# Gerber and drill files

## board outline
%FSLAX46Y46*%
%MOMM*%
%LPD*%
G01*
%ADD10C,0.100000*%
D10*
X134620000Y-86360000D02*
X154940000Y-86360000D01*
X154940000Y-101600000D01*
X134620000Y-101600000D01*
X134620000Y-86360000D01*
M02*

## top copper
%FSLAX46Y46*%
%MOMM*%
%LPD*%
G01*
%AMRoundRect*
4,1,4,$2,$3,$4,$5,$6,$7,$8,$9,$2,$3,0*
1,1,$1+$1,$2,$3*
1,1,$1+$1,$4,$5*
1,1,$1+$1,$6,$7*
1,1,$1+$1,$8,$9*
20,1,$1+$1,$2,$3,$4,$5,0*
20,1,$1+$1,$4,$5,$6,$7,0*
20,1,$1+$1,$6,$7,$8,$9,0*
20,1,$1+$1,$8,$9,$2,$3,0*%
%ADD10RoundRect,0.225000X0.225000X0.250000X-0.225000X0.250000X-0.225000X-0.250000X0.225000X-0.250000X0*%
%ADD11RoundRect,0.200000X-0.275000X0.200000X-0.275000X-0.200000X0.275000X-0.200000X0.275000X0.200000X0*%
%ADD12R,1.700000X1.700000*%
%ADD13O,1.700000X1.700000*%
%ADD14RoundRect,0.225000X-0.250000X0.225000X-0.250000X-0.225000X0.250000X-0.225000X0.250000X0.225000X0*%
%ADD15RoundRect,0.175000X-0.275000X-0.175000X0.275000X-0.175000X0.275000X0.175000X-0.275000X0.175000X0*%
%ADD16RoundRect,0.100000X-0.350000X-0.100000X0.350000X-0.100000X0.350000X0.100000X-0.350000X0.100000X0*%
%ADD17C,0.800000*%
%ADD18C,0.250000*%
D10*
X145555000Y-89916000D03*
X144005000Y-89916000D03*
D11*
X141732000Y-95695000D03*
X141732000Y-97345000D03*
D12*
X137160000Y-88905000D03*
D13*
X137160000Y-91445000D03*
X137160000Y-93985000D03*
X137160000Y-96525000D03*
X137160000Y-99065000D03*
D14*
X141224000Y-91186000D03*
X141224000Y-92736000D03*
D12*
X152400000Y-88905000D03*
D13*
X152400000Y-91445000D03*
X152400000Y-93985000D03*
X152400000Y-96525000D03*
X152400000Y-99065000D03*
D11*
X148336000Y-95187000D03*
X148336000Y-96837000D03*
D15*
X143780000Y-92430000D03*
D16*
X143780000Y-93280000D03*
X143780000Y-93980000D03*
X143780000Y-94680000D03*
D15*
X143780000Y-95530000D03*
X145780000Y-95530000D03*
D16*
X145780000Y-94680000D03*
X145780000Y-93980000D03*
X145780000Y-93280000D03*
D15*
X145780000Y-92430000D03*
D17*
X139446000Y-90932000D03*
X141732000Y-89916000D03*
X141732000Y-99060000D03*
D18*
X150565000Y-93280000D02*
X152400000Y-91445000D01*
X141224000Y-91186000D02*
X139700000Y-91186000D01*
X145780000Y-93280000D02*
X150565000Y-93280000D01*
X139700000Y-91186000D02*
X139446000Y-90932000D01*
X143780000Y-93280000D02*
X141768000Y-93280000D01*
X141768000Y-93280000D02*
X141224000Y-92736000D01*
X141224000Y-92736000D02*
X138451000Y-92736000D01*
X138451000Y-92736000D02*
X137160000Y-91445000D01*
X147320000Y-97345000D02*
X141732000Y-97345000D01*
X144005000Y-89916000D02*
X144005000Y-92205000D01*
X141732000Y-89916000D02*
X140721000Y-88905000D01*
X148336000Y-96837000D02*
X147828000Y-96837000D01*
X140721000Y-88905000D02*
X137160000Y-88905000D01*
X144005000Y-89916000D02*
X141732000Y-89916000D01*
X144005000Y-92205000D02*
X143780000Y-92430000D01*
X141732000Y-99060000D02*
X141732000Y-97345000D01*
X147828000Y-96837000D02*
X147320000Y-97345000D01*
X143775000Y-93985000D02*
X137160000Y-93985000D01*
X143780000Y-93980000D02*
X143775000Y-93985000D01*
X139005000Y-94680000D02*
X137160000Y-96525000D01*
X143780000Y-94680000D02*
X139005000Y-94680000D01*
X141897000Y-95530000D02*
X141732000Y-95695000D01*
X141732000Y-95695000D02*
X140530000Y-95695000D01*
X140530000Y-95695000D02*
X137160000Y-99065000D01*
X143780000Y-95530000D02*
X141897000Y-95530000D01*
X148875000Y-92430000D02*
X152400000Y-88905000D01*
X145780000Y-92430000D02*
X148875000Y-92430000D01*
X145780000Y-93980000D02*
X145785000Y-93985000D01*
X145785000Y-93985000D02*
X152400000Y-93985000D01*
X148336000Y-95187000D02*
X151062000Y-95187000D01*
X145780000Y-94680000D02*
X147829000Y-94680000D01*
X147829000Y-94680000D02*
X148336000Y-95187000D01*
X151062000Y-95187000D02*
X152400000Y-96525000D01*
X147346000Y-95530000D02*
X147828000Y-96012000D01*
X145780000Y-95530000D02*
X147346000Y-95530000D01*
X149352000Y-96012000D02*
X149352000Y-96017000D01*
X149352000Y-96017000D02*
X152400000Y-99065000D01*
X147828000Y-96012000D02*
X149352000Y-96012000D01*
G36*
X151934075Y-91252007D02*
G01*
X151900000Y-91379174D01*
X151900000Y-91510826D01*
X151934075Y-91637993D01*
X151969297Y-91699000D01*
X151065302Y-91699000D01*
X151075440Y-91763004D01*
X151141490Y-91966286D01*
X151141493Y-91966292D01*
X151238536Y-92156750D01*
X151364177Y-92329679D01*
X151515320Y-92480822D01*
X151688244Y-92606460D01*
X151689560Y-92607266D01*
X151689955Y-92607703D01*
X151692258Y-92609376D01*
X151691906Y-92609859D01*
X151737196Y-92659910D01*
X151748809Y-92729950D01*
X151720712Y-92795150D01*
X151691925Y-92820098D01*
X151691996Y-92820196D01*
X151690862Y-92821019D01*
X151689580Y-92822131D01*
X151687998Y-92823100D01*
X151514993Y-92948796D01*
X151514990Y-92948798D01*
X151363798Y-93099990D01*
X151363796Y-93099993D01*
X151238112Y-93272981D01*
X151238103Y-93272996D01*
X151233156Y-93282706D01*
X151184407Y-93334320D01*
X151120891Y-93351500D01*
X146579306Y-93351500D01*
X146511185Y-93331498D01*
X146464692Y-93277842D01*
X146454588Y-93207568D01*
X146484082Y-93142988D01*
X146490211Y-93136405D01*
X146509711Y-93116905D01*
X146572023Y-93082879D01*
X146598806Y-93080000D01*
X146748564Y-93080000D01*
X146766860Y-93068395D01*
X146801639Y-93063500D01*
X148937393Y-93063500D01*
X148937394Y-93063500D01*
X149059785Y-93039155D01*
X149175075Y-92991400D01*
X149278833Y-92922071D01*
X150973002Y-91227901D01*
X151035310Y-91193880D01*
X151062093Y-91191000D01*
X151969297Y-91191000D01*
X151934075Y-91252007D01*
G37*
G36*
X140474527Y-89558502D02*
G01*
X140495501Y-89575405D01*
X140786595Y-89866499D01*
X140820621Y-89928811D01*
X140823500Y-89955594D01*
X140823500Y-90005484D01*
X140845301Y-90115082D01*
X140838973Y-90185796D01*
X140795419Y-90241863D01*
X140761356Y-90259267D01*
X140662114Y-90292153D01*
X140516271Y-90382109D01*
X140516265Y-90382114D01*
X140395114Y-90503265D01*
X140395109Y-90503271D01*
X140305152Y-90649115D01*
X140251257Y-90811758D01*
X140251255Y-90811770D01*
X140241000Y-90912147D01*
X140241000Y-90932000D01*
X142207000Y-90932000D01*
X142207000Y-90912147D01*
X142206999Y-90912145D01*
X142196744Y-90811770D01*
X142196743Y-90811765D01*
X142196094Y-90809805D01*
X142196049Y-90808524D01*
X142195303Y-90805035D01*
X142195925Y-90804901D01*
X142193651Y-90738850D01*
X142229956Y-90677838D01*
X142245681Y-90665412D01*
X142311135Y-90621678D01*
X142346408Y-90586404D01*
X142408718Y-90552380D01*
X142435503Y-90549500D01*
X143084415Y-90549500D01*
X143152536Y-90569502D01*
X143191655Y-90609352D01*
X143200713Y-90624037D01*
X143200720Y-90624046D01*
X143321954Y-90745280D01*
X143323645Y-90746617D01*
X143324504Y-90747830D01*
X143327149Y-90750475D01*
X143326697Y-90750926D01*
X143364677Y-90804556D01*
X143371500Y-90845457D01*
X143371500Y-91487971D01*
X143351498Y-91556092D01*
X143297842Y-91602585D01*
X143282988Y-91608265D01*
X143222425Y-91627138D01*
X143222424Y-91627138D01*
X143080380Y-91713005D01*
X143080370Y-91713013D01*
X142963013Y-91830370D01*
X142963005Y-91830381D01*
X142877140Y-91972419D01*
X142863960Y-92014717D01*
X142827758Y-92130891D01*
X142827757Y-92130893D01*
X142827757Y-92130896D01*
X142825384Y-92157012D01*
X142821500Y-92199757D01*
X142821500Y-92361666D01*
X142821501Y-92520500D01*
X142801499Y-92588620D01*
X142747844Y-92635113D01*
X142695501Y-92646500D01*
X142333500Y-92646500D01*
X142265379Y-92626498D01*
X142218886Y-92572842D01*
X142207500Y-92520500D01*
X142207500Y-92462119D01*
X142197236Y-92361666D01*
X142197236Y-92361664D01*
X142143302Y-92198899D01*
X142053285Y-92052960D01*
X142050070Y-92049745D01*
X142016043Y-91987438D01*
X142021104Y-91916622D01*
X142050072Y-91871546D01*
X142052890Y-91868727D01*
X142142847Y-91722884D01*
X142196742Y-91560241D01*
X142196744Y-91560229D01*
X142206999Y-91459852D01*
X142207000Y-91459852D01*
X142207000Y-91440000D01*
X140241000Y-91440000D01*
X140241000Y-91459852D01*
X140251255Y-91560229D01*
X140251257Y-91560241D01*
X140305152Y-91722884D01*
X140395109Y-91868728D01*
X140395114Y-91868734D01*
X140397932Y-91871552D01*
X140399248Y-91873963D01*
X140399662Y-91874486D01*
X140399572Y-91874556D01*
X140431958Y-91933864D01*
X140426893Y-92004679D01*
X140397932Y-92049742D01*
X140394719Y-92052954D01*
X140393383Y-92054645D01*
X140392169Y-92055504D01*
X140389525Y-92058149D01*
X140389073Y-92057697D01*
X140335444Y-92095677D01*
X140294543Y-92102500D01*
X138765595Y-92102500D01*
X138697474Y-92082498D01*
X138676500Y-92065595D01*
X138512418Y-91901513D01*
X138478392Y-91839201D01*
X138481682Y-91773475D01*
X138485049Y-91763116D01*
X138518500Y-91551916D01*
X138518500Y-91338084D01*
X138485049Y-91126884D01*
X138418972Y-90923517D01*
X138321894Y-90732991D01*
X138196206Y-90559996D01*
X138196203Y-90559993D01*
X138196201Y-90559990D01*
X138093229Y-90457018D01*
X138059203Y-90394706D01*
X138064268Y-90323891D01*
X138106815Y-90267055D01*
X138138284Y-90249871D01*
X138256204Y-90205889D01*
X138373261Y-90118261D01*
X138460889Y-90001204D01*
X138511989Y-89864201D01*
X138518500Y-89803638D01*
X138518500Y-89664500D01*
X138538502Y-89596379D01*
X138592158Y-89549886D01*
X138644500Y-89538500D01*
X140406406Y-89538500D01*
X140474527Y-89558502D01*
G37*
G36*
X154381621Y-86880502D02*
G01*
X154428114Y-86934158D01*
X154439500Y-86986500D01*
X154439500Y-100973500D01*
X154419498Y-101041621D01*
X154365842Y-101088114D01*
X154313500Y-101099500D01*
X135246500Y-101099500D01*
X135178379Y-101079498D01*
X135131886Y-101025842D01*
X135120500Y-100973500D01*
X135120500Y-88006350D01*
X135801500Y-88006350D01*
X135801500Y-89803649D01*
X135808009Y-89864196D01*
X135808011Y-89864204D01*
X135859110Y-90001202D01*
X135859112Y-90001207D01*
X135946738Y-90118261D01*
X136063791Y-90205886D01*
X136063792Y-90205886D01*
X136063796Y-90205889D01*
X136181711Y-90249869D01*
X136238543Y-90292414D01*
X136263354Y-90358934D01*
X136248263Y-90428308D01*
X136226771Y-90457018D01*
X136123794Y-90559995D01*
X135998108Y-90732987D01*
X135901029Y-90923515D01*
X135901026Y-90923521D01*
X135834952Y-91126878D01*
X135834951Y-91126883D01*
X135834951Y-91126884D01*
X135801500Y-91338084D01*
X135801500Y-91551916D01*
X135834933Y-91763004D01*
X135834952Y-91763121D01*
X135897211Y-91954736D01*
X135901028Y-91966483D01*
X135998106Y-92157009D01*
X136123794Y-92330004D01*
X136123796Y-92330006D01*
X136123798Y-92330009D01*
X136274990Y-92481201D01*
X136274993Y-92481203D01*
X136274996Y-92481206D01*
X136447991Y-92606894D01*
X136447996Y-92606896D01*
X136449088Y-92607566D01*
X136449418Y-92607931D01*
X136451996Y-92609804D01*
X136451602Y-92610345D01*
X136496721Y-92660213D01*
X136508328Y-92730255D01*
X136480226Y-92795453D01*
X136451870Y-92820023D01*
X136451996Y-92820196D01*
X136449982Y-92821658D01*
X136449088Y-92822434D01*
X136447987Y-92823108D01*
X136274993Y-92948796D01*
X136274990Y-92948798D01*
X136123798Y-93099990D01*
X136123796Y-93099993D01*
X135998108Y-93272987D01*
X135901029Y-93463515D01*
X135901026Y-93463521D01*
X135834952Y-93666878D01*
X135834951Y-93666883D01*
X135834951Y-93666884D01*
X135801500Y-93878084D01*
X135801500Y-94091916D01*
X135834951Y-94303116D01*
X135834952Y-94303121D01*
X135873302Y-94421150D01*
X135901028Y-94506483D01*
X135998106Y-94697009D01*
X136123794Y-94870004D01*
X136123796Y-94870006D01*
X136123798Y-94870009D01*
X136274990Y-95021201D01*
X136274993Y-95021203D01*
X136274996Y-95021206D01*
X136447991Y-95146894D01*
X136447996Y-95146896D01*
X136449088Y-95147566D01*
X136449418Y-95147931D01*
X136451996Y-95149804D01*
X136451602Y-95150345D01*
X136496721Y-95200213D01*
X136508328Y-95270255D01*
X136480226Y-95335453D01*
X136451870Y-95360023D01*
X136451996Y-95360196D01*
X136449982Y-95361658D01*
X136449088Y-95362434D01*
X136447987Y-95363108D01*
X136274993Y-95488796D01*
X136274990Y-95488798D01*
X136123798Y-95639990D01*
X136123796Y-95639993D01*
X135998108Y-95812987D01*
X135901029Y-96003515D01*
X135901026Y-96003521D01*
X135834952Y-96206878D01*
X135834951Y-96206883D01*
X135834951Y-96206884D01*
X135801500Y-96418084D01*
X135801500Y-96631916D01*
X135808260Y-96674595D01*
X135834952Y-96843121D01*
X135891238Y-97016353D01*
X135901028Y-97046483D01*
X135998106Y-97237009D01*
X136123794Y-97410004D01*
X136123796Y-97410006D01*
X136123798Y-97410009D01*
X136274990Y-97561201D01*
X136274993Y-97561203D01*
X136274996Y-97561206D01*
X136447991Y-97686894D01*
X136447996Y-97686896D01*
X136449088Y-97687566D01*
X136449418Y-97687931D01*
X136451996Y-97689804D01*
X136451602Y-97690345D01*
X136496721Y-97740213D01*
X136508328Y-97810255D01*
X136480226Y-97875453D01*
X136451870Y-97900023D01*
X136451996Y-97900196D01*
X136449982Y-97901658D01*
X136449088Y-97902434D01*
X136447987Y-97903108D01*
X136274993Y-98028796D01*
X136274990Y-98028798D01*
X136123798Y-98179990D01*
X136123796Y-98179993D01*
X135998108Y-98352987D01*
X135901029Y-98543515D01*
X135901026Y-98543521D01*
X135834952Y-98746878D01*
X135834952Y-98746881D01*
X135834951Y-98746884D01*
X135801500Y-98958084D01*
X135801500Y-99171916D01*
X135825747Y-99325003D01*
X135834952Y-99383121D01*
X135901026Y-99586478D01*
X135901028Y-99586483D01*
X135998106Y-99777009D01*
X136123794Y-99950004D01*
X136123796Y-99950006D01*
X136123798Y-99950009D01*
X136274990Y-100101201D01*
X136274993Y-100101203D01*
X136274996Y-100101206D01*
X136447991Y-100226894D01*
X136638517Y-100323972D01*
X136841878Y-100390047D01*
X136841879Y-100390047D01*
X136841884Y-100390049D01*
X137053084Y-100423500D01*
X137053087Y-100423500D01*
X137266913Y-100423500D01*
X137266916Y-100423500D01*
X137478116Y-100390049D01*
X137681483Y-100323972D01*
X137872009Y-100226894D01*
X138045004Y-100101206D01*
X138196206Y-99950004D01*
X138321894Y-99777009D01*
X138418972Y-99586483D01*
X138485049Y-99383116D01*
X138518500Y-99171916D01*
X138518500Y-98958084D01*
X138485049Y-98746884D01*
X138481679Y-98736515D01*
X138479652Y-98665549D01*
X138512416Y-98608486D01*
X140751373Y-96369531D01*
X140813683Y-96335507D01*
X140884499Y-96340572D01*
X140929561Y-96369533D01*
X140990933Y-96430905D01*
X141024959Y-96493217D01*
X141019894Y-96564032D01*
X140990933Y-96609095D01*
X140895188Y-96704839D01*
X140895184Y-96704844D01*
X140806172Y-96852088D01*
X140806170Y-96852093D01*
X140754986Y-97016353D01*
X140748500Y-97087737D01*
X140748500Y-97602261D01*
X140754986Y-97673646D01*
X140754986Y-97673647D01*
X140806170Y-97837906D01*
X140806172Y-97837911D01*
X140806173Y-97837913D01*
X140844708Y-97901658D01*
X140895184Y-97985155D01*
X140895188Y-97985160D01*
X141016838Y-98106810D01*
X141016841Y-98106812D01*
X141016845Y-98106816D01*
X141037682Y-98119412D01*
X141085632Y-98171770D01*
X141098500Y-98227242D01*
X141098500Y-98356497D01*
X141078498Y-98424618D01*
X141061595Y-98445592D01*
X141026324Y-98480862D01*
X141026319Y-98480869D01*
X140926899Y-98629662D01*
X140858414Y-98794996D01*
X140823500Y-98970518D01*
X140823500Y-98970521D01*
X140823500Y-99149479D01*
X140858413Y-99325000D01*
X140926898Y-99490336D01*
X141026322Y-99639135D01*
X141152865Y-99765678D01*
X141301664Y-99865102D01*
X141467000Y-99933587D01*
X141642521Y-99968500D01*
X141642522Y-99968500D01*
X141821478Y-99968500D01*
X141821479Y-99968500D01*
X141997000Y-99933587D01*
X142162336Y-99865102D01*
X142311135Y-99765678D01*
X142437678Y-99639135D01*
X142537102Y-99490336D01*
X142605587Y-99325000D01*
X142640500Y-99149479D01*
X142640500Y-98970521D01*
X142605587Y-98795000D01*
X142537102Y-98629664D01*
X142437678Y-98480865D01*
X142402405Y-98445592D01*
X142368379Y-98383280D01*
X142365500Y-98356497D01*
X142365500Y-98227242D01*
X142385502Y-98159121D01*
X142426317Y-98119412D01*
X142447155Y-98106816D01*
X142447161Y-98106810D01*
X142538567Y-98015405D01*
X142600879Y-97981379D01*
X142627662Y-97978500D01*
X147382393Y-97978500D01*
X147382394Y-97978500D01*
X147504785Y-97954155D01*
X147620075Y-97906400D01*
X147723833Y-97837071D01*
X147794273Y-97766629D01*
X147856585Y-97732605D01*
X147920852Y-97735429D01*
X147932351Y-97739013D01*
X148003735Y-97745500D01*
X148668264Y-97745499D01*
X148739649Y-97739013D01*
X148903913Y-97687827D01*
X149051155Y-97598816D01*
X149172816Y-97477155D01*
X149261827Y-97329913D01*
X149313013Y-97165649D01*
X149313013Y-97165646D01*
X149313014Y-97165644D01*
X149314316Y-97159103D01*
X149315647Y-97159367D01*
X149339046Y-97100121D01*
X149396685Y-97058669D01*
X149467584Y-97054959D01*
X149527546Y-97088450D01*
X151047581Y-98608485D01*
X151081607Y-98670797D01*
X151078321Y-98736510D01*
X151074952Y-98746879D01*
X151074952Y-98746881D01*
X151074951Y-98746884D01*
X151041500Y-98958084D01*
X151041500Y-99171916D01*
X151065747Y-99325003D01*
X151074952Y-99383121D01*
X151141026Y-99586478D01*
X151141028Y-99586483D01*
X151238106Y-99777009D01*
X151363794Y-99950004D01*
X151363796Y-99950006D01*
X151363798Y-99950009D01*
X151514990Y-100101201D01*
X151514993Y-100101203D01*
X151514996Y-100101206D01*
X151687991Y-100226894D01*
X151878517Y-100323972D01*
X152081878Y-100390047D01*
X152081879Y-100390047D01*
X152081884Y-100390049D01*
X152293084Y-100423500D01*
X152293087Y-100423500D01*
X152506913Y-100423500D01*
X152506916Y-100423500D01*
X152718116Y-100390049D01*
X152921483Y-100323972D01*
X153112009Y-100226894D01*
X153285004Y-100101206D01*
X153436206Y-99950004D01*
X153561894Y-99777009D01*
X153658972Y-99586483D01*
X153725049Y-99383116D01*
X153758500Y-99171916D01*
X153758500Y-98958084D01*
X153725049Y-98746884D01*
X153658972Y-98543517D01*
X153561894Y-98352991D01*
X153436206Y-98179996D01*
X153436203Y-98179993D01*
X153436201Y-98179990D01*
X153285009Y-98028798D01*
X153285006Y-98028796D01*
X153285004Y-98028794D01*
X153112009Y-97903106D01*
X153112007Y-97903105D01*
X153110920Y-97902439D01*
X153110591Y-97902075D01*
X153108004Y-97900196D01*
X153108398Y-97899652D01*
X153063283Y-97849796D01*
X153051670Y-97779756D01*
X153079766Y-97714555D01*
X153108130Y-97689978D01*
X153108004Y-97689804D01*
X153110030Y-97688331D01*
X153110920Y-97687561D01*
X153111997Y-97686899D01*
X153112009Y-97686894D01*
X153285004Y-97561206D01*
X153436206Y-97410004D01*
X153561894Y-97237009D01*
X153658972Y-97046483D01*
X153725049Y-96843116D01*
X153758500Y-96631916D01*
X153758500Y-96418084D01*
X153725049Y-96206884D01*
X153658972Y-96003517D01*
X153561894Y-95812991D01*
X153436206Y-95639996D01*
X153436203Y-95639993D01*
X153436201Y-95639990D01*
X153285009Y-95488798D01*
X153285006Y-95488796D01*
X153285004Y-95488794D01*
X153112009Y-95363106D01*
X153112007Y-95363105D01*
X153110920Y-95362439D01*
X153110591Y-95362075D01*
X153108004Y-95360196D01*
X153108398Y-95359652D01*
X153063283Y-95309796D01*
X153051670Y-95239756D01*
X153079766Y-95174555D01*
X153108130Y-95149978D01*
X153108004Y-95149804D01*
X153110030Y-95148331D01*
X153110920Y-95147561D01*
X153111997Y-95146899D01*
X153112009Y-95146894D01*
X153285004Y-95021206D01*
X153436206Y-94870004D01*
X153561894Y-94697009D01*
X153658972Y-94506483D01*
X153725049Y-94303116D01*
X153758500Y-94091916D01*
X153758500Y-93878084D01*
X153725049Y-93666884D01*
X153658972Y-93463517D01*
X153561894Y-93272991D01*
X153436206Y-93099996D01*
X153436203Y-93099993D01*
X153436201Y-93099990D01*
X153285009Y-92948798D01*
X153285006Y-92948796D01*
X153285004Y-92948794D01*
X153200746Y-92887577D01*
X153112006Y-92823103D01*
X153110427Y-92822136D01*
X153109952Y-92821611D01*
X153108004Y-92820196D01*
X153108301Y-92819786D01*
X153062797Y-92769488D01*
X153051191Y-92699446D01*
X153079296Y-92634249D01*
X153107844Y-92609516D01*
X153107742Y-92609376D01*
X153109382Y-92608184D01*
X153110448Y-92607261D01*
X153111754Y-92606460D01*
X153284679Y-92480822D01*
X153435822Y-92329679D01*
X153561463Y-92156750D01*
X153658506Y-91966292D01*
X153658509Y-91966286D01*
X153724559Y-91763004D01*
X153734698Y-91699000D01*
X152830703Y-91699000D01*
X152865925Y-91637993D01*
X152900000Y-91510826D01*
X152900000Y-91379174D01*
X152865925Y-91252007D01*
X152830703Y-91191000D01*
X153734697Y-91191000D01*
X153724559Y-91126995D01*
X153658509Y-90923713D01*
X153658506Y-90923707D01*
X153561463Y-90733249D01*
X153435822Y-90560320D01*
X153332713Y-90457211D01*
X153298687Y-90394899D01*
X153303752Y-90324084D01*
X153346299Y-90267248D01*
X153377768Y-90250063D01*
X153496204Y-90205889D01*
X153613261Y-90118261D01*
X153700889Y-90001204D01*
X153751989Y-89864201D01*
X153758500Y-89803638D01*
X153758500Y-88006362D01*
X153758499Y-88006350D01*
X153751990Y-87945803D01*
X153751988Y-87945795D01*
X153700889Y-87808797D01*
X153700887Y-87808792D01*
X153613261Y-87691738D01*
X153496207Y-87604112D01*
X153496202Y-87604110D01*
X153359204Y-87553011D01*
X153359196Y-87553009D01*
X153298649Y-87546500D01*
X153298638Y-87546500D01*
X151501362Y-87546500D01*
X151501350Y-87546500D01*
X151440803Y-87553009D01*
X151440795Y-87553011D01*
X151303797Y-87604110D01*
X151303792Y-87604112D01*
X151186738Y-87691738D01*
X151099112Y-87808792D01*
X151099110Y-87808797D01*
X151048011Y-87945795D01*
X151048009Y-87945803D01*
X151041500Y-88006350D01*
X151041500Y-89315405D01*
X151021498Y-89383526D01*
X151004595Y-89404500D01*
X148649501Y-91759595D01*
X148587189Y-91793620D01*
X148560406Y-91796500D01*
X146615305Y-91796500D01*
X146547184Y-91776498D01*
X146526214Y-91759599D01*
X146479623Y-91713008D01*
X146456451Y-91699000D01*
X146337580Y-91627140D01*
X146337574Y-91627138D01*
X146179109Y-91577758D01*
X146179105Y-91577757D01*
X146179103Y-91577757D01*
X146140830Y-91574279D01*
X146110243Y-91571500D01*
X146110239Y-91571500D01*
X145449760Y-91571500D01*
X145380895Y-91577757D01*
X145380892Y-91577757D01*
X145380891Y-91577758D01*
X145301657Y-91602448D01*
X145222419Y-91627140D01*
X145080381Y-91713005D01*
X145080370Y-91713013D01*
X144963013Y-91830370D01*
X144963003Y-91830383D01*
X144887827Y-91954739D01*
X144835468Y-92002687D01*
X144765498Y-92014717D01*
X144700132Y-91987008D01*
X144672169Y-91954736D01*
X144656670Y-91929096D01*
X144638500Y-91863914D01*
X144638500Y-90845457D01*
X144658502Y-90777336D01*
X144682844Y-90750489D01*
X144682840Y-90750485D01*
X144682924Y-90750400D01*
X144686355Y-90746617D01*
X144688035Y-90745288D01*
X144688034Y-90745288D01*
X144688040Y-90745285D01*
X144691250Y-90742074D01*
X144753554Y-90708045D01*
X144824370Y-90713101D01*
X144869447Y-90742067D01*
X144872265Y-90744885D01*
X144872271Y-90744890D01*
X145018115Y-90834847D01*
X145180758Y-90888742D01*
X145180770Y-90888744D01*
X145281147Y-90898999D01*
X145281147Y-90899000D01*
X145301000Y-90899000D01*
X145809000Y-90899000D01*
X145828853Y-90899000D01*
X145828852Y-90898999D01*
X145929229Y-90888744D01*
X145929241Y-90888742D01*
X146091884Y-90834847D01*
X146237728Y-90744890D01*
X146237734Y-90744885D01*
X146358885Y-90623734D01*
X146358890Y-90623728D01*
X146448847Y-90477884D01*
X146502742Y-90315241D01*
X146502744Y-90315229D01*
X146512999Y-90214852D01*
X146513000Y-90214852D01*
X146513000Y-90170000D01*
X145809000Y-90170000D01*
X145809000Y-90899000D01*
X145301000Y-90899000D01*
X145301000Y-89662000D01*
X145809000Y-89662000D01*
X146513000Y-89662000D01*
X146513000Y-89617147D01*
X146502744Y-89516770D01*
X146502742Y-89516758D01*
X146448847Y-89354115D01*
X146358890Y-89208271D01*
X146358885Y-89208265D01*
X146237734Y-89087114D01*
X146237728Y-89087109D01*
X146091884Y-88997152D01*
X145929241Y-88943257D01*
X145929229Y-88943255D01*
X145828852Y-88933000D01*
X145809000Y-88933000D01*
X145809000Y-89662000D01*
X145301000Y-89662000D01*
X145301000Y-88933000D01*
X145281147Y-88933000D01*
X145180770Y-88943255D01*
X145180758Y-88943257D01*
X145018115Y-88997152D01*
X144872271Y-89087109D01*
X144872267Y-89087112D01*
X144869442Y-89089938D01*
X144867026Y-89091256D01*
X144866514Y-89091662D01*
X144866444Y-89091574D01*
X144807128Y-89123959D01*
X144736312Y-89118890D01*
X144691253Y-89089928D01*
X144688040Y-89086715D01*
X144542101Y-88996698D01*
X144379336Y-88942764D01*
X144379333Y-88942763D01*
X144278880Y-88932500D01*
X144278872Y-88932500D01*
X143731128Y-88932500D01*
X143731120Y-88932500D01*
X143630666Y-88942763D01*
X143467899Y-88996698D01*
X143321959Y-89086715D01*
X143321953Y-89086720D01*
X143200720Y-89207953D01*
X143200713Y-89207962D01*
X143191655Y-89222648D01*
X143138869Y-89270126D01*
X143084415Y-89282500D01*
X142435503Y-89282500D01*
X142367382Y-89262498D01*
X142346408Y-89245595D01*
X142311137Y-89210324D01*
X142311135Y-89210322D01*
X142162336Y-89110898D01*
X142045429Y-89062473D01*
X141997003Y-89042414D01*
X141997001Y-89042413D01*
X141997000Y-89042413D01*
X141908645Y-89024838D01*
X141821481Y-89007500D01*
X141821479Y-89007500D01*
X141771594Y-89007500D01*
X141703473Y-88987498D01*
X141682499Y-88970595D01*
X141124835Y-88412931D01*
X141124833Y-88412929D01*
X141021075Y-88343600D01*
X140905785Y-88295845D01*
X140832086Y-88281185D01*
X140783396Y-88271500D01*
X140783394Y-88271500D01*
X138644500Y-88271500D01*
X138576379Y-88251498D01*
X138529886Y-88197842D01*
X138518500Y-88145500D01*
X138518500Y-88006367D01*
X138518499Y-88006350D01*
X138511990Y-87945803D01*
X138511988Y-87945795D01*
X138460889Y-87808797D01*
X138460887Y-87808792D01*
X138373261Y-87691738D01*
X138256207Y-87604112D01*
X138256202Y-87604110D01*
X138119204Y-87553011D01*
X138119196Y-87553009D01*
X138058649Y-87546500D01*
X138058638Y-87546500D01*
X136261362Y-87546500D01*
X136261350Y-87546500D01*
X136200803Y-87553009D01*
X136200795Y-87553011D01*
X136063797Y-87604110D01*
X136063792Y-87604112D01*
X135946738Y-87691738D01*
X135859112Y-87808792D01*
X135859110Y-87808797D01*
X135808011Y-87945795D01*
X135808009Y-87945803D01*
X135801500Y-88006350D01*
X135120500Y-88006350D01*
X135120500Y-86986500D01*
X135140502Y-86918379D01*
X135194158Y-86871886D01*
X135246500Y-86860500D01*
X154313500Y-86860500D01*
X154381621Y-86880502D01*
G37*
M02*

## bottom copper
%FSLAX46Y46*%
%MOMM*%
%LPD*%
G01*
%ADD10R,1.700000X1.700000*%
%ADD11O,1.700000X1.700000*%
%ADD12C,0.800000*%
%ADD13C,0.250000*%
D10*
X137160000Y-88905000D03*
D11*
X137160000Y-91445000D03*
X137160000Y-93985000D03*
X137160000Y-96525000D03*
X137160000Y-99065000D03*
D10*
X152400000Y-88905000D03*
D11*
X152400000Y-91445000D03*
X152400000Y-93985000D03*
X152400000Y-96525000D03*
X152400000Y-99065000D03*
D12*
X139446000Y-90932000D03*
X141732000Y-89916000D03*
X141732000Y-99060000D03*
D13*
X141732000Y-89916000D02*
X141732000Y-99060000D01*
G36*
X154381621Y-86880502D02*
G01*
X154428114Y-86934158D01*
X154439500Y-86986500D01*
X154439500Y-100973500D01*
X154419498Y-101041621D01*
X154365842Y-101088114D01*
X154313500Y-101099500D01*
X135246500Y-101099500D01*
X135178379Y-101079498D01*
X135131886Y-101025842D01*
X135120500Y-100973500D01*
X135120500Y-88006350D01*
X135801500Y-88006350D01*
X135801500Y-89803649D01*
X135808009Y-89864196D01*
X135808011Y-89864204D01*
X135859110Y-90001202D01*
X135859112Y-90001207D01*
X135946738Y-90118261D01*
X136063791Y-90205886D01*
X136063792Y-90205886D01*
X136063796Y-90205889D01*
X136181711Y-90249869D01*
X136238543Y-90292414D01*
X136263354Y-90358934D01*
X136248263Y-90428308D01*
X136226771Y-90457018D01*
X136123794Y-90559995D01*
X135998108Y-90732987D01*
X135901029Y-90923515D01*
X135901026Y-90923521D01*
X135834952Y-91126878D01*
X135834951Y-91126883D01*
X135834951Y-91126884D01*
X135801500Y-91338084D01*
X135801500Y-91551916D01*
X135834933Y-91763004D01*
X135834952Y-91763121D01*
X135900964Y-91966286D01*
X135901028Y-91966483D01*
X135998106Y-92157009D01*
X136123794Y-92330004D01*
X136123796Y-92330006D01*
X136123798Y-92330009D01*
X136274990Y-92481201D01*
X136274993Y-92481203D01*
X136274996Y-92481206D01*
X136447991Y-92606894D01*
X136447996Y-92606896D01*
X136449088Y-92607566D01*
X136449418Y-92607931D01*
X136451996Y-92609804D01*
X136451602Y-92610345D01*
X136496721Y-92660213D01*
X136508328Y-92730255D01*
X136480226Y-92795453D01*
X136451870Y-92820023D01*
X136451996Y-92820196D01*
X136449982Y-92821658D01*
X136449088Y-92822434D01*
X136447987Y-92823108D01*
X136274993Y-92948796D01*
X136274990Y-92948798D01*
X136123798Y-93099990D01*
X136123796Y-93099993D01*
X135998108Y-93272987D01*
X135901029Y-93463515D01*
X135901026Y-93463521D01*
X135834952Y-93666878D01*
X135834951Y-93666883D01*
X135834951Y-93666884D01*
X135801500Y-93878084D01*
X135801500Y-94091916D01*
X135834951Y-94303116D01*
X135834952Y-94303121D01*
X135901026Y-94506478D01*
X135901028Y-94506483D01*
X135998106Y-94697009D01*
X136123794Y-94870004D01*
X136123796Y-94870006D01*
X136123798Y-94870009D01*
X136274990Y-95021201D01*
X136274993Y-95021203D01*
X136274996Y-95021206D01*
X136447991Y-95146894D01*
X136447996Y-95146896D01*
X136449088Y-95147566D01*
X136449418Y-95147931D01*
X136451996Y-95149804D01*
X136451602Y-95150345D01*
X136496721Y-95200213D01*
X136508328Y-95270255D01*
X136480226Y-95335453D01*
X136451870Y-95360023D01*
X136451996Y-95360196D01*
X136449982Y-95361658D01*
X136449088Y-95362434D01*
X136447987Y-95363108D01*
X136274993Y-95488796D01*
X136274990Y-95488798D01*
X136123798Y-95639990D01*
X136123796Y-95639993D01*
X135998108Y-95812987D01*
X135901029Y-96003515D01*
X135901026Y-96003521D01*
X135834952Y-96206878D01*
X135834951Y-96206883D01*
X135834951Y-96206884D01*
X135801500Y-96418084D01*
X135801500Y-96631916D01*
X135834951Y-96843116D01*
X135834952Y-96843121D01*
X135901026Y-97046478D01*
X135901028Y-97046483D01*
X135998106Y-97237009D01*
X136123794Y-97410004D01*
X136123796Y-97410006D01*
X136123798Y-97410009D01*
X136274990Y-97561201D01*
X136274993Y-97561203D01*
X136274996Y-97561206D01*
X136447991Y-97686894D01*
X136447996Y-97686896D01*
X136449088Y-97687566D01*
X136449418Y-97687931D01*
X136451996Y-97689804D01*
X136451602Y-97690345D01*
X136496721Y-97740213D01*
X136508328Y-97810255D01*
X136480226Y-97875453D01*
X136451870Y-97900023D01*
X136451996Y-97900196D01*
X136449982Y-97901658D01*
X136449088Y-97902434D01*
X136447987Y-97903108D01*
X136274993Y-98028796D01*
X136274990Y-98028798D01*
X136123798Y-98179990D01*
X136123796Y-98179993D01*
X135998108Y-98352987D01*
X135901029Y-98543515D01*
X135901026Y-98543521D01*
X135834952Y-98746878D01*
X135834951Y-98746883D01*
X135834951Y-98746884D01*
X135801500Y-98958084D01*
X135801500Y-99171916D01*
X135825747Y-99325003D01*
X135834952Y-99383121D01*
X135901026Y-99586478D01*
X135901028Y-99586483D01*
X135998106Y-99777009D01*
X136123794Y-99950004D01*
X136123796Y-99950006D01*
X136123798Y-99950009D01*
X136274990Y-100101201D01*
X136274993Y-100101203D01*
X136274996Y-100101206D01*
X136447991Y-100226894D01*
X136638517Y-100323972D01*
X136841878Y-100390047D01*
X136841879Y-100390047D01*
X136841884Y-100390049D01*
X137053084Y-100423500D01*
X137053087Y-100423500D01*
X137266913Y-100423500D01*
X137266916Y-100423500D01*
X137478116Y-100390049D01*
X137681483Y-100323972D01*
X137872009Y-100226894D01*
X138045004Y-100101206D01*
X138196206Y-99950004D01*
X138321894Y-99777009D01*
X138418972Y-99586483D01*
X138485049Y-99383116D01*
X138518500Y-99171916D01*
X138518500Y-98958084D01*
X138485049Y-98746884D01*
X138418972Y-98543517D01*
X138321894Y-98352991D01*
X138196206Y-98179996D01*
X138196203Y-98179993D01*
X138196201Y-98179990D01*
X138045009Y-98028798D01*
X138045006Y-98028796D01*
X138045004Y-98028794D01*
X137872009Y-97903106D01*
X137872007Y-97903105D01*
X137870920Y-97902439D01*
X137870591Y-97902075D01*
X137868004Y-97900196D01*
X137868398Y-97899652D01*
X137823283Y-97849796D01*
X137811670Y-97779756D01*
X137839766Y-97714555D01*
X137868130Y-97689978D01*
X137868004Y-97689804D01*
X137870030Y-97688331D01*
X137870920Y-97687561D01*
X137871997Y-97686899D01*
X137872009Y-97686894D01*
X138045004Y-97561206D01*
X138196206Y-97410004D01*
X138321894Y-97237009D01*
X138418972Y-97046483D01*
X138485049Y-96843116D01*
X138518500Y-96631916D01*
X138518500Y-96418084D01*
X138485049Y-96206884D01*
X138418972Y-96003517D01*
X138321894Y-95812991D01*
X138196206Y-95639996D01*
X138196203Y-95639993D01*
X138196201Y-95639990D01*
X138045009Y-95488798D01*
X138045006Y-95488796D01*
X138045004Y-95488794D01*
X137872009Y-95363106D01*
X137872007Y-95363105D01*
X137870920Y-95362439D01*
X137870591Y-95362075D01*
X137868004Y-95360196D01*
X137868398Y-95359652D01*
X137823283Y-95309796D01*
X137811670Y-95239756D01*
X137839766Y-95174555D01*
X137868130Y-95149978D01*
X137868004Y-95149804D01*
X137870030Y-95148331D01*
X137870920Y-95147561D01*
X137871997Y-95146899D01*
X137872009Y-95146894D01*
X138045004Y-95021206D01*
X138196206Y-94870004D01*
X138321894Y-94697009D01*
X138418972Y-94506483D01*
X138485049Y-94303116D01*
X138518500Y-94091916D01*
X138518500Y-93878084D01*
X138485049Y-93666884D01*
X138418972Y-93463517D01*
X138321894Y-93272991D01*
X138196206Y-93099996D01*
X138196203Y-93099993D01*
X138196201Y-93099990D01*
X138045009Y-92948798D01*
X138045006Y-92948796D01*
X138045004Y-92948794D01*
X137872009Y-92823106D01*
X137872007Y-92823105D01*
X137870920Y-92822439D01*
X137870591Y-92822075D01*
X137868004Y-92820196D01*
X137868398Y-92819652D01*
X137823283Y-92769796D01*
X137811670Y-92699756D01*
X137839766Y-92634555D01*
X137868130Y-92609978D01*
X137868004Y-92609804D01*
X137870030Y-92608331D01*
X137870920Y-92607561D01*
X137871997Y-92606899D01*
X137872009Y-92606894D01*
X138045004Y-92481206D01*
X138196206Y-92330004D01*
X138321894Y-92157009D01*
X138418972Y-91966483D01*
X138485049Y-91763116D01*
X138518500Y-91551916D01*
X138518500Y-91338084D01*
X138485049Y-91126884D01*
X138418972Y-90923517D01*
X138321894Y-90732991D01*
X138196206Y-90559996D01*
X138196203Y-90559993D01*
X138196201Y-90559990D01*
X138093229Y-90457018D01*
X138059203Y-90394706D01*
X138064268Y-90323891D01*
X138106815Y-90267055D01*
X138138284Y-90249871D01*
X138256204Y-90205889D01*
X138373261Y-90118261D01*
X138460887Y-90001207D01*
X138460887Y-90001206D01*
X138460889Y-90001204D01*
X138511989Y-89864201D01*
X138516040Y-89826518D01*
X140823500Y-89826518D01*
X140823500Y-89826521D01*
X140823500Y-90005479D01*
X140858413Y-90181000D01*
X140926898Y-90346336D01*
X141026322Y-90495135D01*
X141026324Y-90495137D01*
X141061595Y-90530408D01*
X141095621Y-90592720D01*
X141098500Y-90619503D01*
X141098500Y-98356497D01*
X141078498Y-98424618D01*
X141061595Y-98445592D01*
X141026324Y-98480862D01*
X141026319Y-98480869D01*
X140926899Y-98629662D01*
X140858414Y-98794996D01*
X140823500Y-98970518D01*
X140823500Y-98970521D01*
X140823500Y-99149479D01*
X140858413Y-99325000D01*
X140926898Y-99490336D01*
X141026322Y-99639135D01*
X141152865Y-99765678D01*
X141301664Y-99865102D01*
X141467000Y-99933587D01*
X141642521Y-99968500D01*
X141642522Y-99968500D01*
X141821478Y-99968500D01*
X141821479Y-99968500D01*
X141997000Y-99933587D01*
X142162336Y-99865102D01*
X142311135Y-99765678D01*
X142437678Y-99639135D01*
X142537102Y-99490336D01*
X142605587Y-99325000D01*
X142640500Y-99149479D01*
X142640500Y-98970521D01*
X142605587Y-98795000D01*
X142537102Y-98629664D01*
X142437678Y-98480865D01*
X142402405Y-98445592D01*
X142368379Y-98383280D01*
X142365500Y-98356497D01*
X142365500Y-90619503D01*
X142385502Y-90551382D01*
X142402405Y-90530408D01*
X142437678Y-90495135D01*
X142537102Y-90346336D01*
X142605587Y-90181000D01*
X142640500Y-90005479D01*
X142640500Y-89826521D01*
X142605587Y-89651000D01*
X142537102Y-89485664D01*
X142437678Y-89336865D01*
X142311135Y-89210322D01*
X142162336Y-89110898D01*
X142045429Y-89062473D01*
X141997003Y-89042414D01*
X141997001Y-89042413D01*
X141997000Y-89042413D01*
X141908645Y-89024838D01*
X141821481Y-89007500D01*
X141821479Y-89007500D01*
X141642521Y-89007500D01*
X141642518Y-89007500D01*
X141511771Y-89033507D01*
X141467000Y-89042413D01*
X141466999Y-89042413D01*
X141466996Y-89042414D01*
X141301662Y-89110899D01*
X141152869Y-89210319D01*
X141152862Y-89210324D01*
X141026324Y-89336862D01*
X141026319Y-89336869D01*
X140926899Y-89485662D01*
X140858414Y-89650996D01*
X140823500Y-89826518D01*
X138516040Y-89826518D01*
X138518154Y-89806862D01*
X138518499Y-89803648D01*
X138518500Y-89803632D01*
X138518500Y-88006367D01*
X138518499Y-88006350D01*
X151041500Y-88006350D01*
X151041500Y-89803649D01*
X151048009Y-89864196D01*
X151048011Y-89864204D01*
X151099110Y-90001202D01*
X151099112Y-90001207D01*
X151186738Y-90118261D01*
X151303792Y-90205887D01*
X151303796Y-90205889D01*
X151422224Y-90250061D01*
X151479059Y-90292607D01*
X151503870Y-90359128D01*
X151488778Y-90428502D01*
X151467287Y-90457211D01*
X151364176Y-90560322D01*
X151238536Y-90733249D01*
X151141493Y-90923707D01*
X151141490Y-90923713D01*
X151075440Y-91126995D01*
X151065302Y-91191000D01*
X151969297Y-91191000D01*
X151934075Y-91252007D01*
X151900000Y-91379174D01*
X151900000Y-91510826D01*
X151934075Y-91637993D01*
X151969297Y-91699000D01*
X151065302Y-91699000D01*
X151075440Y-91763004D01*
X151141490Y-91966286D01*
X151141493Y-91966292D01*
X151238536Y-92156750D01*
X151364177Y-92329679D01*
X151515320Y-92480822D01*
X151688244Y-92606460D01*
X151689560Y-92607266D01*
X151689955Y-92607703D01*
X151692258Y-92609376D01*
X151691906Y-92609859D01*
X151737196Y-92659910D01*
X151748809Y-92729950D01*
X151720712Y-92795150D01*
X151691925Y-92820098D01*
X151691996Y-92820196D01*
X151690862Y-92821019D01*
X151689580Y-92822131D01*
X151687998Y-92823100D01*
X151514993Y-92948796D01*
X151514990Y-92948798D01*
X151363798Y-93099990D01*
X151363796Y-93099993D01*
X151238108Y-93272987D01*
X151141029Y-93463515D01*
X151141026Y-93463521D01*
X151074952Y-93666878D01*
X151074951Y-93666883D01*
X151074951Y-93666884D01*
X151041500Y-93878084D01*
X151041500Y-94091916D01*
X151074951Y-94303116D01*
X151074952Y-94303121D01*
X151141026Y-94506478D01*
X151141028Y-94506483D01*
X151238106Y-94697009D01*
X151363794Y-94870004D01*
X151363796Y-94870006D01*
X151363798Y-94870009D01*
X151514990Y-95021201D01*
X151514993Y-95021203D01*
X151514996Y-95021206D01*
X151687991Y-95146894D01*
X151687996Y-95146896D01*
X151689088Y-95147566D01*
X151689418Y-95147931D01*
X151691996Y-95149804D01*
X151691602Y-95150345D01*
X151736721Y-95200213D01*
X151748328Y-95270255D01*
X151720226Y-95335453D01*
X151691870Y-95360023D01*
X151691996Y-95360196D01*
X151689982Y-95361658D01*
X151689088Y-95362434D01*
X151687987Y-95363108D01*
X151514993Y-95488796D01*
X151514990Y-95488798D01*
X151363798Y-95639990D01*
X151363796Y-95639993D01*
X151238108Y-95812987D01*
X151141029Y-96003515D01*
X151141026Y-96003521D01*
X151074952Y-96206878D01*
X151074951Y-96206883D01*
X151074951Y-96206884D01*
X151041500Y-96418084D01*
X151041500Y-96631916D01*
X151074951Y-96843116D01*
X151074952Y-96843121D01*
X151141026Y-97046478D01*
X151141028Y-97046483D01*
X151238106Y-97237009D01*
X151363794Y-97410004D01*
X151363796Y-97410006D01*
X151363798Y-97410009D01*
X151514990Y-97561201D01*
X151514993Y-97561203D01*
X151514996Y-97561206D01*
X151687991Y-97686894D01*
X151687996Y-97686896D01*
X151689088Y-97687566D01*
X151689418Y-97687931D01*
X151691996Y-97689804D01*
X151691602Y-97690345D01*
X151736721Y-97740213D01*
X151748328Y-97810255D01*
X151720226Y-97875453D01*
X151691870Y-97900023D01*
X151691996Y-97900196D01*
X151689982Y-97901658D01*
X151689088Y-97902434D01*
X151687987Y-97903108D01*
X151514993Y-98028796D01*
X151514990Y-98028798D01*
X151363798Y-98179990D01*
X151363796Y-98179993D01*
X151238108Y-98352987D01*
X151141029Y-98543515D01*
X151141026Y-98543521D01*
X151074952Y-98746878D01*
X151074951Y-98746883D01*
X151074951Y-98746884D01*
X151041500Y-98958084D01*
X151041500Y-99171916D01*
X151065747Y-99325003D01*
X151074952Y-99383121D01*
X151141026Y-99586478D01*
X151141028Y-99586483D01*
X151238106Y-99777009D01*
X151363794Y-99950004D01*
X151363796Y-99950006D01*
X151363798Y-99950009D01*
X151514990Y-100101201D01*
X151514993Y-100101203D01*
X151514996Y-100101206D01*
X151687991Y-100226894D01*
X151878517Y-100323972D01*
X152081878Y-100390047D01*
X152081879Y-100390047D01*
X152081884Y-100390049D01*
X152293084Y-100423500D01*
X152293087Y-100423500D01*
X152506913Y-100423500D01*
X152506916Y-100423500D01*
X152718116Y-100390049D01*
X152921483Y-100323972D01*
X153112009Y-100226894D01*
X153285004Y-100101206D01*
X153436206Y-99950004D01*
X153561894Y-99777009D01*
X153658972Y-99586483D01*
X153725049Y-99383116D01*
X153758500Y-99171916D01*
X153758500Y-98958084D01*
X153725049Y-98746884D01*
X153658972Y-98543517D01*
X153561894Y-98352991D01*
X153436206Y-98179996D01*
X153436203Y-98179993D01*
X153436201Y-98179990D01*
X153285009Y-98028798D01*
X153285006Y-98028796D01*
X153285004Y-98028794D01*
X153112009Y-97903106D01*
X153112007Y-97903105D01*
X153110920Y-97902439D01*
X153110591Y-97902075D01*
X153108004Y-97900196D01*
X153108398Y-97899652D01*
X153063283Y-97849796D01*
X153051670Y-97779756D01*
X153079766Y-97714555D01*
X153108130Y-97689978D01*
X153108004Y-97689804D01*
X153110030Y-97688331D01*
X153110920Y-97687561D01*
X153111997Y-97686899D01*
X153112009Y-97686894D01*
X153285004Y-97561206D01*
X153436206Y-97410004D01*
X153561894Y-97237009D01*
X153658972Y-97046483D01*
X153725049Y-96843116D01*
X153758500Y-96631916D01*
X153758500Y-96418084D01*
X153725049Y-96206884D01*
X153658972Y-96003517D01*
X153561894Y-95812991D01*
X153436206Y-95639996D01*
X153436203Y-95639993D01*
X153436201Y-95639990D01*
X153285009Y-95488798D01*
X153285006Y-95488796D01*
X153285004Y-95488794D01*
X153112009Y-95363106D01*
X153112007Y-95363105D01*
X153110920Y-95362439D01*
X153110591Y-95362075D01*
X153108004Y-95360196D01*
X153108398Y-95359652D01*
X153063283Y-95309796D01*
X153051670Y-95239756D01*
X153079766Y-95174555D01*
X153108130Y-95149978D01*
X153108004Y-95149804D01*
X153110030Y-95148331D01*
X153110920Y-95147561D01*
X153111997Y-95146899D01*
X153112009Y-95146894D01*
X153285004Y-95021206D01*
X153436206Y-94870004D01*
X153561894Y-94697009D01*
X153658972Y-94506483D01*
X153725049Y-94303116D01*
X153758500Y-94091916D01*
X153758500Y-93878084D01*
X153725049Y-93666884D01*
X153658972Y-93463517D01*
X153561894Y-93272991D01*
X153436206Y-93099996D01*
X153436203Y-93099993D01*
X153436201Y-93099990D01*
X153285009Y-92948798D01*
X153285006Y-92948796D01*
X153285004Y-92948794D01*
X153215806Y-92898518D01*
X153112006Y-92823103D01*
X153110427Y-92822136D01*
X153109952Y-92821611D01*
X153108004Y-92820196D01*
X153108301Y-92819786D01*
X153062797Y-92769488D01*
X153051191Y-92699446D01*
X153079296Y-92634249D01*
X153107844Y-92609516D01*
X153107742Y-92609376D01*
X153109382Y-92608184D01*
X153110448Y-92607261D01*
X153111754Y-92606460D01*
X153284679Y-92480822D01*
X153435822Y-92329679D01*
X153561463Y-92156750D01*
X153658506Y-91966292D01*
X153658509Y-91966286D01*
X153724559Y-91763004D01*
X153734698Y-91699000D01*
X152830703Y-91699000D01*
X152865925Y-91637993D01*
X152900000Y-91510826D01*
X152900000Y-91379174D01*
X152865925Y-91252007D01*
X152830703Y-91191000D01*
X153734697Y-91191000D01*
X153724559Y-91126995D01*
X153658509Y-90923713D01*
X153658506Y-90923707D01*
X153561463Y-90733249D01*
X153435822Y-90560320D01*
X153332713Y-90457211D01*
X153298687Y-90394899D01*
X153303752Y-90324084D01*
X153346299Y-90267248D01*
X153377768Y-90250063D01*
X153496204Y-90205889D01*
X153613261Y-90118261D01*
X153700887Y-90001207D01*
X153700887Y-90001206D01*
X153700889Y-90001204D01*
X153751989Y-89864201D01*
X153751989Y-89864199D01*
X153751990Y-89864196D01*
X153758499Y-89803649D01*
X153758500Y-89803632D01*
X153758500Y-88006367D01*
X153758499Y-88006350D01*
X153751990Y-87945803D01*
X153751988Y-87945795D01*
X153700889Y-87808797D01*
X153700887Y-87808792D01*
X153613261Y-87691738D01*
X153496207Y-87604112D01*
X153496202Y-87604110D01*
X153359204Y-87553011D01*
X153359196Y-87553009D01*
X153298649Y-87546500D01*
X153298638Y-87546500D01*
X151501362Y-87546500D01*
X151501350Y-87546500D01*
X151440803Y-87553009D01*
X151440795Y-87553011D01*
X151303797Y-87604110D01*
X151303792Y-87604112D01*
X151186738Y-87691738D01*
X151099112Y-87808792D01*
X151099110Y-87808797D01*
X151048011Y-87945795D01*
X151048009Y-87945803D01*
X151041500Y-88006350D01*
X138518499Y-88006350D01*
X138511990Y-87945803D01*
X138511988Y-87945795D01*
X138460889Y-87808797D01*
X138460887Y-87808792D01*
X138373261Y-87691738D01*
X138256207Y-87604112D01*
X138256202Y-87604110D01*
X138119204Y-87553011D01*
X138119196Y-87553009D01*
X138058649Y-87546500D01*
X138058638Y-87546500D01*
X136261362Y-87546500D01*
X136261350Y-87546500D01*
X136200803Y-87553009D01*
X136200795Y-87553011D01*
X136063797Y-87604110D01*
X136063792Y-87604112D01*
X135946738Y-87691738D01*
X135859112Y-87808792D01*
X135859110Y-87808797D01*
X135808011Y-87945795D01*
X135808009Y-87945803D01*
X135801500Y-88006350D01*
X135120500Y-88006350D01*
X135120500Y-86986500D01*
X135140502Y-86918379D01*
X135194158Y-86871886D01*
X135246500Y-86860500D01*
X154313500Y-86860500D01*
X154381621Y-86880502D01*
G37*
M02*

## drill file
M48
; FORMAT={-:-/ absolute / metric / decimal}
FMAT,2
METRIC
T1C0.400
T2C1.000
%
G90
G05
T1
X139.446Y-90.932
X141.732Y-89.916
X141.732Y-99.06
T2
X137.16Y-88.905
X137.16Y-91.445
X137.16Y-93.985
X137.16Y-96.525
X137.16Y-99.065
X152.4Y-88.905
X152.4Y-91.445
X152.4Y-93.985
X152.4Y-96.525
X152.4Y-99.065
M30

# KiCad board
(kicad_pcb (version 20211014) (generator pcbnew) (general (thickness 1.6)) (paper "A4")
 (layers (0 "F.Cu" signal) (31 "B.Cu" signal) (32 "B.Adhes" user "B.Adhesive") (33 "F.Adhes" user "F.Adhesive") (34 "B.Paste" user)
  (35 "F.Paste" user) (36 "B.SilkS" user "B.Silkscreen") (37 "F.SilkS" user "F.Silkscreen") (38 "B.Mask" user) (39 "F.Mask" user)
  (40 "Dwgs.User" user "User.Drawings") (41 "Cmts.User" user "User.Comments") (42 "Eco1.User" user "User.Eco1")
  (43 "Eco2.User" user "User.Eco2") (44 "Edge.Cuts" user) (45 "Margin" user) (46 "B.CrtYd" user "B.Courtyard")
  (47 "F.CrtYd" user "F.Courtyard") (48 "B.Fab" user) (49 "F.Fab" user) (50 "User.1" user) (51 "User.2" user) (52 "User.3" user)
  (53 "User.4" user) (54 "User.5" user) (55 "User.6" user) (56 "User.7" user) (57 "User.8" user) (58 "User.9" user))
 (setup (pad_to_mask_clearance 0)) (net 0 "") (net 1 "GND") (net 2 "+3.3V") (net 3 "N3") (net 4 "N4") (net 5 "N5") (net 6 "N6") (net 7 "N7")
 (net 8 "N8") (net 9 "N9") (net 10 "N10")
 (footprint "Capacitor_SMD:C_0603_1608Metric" (layer "F.Cu") (at 144.78 89.916 180)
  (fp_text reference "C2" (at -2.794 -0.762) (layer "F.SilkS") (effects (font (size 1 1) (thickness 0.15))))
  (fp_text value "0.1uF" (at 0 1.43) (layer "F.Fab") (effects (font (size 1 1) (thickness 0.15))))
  (pad "1" smd roundrect (at -0.775 0 180) (size 0.9 0.95) (layers "F.Cu" "F.Paste" "F.Mask") (roundrect_rratio 0.25) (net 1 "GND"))
  (pad "2" smd roundrect (at 0.775 0 180) (size 0.9 0.95) (layers "F.Cu" "F.Paste" "F.Mask") (roundrect_rratio 0.25) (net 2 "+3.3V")))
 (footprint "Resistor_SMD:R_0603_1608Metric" (layer "F.Cu") (at 141.732 96.52 -90)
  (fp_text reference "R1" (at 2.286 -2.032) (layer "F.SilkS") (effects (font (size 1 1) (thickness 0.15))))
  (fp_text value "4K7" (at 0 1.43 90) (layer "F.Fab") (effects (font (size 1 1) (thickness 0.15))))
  (pad "1" smd roundrect (at -0.825 0 270) (size 0.8 0.95) (layers "F.Cu" "F.Paste" "F.Mask") (roundrect_rratio 0.25) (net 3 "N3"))
  (pad "2" smd roundrect (at 0.825 0 270) (size 0.8 0.95) (layers "F.Cu" "F.Paste" "F.Mask") (roundrect_rratio 0.25) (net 2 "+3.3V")))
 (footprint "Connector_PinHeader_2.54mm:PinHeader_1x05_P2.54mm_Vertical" (layer "F.Cu") (at 137.16 88.905)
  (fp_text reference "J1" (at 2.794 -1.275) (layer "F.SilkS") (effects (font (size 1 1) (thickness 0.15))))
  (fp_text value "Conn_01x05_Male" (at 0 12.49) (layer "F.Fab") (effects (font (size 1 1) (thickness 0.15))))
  (pad "1" thru_hole rect (at 0 0) (size 1.7 1.7) (drill 1) (layers *.Cu *.Mask) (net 2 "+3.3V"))
  (pad "2" thru_hole oval (at 0 2.54) (size 1.7 1.7) (drill 1) (layers *.Cu *.Mask) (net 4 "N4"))
  (pad "3" thru_hole oval (at 0 5.08) (size 1.7 1.7) (drill 1) (layers *.Cu *.Mask) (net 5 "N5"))
  (pad "4" thru_hole oval (at 0 7.62) (size 1.7 1.7) (drill 1) (layers *.Cu *.Mask) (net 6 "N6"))
  (pad "5" thru_hole oval (at 0 10.16) (size 1.7 1.7) (drill 1) (layers *.Cu *.Mask) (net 3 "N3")))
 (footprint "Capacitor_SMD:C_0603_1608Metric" (layer "F.Cu") (at 141.224 91.961 -90)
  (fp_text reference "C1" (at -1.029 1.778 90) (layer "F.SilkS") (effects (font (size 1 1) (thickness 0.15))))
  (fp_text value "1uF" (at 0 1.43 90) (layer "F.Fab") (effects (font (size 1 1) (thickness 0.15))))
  (pad "1" smd roundrect (at -0.775 0 270) (size 0.9 0.95) (layers "F.Cu" "F.Paste" "F.Mask") (roundrect_rratio 0.25) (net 1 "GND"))
  (pad "2" smd roundrect (at 0.775 0 270) (size 0.9 0.95) (layers "F.Cu" "F.Paste" "F.Mask") (roundrect_rratio 0.25) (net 4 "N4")))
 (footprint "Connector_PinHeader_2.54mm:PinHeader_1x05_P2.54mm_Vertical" (layer "F.Cu") (at 152.4 88.905)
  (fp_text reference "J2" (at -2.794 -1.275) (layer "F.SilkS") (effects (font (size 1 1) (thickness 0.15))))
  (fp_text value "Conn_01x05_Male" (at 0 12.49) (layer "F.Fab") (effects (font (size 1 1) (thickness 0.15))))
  (pad "1" thru_hole rect (at 0 0) (size 1.7 1.7) (drill 1) (layers *.Cu *.Mask) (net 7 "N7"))
  (pad "2" thru_hole oval (at 0 2.54) (size 1.7 1.7) (drill 1) (layers *.Cu *.Mask) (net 1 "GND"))
  (pad "3" thru_hole oval (at 0 5.08) (size 1.7 1.7) (drill 1) (layers *.Cu *.Mask) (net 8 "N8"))
  (pad "4" thru_hole oval (at 0 7.62) (size 1.7 1.7) (drill 1) (layers *.Cu *.Mask) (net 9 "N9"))
  (pad "5" thru_hole oval (at 0 10.16) (size 1.7 1.7) (drill 1) (layers *.Cu *.Mask) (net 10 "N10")))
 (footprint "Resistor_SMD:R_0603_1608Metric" (layer "F.Cu") (at 148.336 96.012 -90)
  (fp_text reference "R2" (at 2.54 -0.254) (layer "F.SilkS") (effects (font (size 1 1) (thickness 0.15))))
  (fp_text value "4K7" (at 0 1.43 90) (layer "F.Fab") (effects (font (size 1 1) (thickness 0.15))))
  (pad "1" smd roundrect (at -0.825 0 270) (size 0.8 0.95) (layers "F.Cu" "F.Paste" "F.Mask") (roundrect_rratio 0.25) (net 9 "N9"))
  (pad "2" smd roundrect (at 0.825 0 270) (size 0.8 0.95) (layers "F.Cu" "F.Paste" "F.Mask") (roundrect_rratio 0.25) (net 2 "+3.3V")))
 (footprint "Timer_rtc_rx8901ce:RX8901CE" (layer "F.Cu") (at 144.78 93.98)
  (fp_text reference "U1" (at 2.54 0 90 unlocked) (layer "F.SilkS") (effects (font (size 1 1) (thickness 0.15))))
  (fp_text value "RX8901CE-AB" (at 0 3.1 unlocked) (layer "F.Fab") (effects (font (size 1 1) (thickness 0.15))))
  (pad "1" smd roundrect (at -1 -1.55) (size 0.9 0.7) (layers "F.Cu" "F.Paste" "F.Mask") (roundrect_rratio 0.25) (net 2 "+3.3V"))
  (pad "2" smd roundrect (at -1 -0.7) (size 0.9 0.4) (layers "F.Cu" "F.Paste" "F.Mask") (roundrect_rratio 0.25) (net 4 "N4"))
  (pad "3" smd roundrect (at -1 0) (size 0.9 0.4) (layers "F.Cu" "F.Paste" "F.Mask") (roundrect_rratio 0.25) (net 5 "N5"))
  (pad "4" smd roundrect (at -1 0.7) (size 0.9 0.4) (layers "F.Cu" "F.Paste" "F.Mask") (roundrect_rratio 0.25) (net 6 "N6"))
  (pad "5" smd roundrect (at -1 1.55) (size 0.9 0.7) (layers "F.Cu" "F.Paste" "F.Mask") (roundrect_rratio 0.25) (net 3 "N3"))
  (pad "6" smd roundrect (at 1 1.55) (size 0.9 0.7) (layers "F.Cu" "F.Paste" "F.Mask") (roundrect_rratio 0.25) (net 10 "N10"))
  (pad "7" smd roundrect (at 1 0.7) (size 0.9 0.4) (layers "F.Cu" "F.Paste" "F.Mask") (roundrect_rratio 0.25) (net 9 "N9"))
  (pad "8" smd roundrect (at 1 0) (size 0.9 0.4) (layers "F.Cu" "F.Paste" "F.Mask") (roundrect_rratio 0.25) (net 8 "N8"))
  (pad "9" smd roundrect (at 1 -0.7) (size 0.9 0.4) (layers "F.Cu" "F.Paste" "F.Mask") (roundrect_rratio 0.25) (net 1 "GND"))
  (pad "10" smd roundrect (at 1 -1.55) (size 0.9 0.7) (layers "F.Cu" "F.Paste" "F.Mask") (roundrect_rratio 0.25) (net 7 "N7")))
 (gr_rect (start 134.62 86.36) (end 154.94 101.6) (layer "Edge.Cuts") (width 0.1) (fill none))
 (segment (start 150.565 93.28) (end 152.4 91.445) (width 0.25) (layer "F.Cu") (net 1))
 (segment (start 141.224 91.186) (end 139.7 91.186) (width 0.25) (layer "F.Cu") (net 1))
 (segment (start 145.78 93.28) (end 150.565 93.28) (width 0.25) (layer "F.Cu") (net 1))
 (segment (start 139.7 91.186) (end 139.446 90.932) (width 0.25) (layer "F.Cu") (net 1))
 (via (at 139.446 90.932) (size 0.8) (drill 0.4) (layers "F.Cu" "B.Cu") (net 1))
 (segment (start 143.78 93.28) (end 141.768 93.28) (width 0.25) (layer "F.Cu") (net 4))
 (segment (start 141.768 93.28) (end 141.224 92.736) (width 0.25) (layer "F.Cu") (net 4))
 (segment (start 141.224 92.736) (end 138.451 92.736) (width 0.25) (layer "F.Cu") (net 4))
 (segment (start 138.451 92.736) (end 137.16 91.445) (width 0.25) (layer "F.Cu") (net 4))
 (segment (start 147.32 97.345) (end 141.732 97.345) (width 0.25) (layer "F.Cu") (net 2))
 (segment (start 144.005 89.916) (end 144.005 92.205) (width 0.25) (layer "F.Cu") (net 2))
 (segment (start 141.732 89.916) (end 140.721 88.905) (width 0.25) (layer "F.Cu") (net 2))
 (segment (start 148.336 96.837) (end 147.828 96.837) (width 0.25) (layer "F.Cu") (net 2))
 (segment (start 140.721 88.905) (end 137.16 88.905) (width 0.25) (layer "F.Cu") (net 2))
 (segment (start 144.005 89.916) (end 141.732 89.916) (width 0.25) (layer "F.Cu") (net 2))
 (segment (start 144.005 92.205) (end 143.78 92.43) (width 0.25) (layer "F.Cu") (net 2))
 (segment (start 141.732 99.06) (end 141.732 97.345) (width 0.25) (layer "F.Cu") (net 2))
 (segment (start 147.828 96.837) (end 147.32 97.345) (width 0.25) (layer "F.Cu") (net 2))
 (via (at 141.732 89.916) (size 0.8) (drill 0.4) (layers "F.Cu" "B.Cu") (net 2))
 (via (at 141.732 99.06) (size 0.8) (drill 0.4) (layers "F.Cu" "B.Cu") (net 2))
 (segment (start 141.732 89.916) (end 141.732 99.06) (width 0.25) (layer "B.Cu") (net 2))
 (segment (start 143.775 93.985) (end 137.16 93.985) (width 0.25) (layer "F.Cu") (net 5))
 (segment (start 143.78 93.98) (end 143.775 93.985) (width 0.25) (layer "F.Cu") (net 5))
 (segment (start 139.005 94.68) (end 137.16 96.525) (width 0.25) (layer "F.Cu") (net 6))
 (segment (start 143.78 94.68) (end 139.005 94.68) (width 0.25) (layer "F.Cu") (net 6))
 (segment (start 141.897 95.53) (end 141.732 95.695) (width 0.25) (layer "F.Cu") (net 3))
 (segment (start 141.732 95.695) (end 140.53 95.695) (width 0.25) (layer "F.Cu") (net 3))
 (segment (start 140.53 95.695) (end 137.16 99.065) (width 0.25) (layer "F.Cu") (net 3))
 (segment (start 143.78 95.53) (end 141.897 95.53) (width 0.25) (layer "F.Cu") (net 3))
 (segment (start 148.875 92.43) (end 152.4 88.905) (width 0.25) (layer "F.Cu") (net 7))
 (segment (start 145.78 92.43) (end 148.875 92.43) (width 0.25) (layer "F.Cu") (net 7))
 (segment (start 145.78 93.98) (end 145.785 93.985) (width 0.25) (layer "F.Cu") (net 8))
 (segment (start 145.785 93.985) (end 152.4 93.985) (width 0.25) (layer "F.Cu") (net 8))
 (segment (start 148.336 95.187) (end 151.062 95.187) (width 0.25) (layer "F.Cu") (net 9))
 (segment (start 145.78 94.68) (end 147.829 94.68) (width 0.25) (layer "F.Cu") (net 9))
 (segment (start 147.829 94.68) (end 148.336 95.187) (width 0.25) (layer "F.Cu") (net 9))
 (segment (start 151.062 95.187) (end 152.4 96.525) (width 0.25) (layer "F.Cu") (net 9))
 (segment (start 147.346 95.53) (end 147.828 96.012) (width 0.25) (layer "F.Cu") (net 10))
 (segment (start 145.78 95.53) (end 147.346 95.53) (width 0.25) (layer "F.Cu") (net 10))
 (segment (start 149.352 96.012) (end 149.352 96.017) (width 0.25) (layer "F.Cu") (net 10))
 (segment (start 149.352 96.017) (end 152.4 99.065) (width 0.25) (layer "F.Cu") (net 10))
 (segment (start 147.828 96.012) (end 149.352 96.012) (width 0.25) (layer "F.Cu") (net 10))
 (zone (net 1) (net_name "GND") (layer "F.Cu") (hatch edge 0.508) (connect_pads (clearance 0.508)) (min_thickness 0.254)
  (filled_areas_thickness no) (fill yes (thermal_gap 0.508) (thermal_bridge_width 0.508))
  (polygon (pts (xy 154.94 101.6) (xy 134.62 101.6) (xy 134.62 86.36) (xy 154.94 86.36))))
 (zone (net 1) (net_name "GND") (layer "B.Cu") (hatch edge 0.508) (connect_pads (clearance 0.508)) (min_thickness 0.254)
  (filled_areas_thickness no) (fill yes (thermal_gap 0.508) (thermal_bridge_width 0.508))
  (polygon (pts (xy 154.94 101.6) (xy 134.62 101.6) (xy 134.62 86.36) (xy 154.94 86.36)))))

